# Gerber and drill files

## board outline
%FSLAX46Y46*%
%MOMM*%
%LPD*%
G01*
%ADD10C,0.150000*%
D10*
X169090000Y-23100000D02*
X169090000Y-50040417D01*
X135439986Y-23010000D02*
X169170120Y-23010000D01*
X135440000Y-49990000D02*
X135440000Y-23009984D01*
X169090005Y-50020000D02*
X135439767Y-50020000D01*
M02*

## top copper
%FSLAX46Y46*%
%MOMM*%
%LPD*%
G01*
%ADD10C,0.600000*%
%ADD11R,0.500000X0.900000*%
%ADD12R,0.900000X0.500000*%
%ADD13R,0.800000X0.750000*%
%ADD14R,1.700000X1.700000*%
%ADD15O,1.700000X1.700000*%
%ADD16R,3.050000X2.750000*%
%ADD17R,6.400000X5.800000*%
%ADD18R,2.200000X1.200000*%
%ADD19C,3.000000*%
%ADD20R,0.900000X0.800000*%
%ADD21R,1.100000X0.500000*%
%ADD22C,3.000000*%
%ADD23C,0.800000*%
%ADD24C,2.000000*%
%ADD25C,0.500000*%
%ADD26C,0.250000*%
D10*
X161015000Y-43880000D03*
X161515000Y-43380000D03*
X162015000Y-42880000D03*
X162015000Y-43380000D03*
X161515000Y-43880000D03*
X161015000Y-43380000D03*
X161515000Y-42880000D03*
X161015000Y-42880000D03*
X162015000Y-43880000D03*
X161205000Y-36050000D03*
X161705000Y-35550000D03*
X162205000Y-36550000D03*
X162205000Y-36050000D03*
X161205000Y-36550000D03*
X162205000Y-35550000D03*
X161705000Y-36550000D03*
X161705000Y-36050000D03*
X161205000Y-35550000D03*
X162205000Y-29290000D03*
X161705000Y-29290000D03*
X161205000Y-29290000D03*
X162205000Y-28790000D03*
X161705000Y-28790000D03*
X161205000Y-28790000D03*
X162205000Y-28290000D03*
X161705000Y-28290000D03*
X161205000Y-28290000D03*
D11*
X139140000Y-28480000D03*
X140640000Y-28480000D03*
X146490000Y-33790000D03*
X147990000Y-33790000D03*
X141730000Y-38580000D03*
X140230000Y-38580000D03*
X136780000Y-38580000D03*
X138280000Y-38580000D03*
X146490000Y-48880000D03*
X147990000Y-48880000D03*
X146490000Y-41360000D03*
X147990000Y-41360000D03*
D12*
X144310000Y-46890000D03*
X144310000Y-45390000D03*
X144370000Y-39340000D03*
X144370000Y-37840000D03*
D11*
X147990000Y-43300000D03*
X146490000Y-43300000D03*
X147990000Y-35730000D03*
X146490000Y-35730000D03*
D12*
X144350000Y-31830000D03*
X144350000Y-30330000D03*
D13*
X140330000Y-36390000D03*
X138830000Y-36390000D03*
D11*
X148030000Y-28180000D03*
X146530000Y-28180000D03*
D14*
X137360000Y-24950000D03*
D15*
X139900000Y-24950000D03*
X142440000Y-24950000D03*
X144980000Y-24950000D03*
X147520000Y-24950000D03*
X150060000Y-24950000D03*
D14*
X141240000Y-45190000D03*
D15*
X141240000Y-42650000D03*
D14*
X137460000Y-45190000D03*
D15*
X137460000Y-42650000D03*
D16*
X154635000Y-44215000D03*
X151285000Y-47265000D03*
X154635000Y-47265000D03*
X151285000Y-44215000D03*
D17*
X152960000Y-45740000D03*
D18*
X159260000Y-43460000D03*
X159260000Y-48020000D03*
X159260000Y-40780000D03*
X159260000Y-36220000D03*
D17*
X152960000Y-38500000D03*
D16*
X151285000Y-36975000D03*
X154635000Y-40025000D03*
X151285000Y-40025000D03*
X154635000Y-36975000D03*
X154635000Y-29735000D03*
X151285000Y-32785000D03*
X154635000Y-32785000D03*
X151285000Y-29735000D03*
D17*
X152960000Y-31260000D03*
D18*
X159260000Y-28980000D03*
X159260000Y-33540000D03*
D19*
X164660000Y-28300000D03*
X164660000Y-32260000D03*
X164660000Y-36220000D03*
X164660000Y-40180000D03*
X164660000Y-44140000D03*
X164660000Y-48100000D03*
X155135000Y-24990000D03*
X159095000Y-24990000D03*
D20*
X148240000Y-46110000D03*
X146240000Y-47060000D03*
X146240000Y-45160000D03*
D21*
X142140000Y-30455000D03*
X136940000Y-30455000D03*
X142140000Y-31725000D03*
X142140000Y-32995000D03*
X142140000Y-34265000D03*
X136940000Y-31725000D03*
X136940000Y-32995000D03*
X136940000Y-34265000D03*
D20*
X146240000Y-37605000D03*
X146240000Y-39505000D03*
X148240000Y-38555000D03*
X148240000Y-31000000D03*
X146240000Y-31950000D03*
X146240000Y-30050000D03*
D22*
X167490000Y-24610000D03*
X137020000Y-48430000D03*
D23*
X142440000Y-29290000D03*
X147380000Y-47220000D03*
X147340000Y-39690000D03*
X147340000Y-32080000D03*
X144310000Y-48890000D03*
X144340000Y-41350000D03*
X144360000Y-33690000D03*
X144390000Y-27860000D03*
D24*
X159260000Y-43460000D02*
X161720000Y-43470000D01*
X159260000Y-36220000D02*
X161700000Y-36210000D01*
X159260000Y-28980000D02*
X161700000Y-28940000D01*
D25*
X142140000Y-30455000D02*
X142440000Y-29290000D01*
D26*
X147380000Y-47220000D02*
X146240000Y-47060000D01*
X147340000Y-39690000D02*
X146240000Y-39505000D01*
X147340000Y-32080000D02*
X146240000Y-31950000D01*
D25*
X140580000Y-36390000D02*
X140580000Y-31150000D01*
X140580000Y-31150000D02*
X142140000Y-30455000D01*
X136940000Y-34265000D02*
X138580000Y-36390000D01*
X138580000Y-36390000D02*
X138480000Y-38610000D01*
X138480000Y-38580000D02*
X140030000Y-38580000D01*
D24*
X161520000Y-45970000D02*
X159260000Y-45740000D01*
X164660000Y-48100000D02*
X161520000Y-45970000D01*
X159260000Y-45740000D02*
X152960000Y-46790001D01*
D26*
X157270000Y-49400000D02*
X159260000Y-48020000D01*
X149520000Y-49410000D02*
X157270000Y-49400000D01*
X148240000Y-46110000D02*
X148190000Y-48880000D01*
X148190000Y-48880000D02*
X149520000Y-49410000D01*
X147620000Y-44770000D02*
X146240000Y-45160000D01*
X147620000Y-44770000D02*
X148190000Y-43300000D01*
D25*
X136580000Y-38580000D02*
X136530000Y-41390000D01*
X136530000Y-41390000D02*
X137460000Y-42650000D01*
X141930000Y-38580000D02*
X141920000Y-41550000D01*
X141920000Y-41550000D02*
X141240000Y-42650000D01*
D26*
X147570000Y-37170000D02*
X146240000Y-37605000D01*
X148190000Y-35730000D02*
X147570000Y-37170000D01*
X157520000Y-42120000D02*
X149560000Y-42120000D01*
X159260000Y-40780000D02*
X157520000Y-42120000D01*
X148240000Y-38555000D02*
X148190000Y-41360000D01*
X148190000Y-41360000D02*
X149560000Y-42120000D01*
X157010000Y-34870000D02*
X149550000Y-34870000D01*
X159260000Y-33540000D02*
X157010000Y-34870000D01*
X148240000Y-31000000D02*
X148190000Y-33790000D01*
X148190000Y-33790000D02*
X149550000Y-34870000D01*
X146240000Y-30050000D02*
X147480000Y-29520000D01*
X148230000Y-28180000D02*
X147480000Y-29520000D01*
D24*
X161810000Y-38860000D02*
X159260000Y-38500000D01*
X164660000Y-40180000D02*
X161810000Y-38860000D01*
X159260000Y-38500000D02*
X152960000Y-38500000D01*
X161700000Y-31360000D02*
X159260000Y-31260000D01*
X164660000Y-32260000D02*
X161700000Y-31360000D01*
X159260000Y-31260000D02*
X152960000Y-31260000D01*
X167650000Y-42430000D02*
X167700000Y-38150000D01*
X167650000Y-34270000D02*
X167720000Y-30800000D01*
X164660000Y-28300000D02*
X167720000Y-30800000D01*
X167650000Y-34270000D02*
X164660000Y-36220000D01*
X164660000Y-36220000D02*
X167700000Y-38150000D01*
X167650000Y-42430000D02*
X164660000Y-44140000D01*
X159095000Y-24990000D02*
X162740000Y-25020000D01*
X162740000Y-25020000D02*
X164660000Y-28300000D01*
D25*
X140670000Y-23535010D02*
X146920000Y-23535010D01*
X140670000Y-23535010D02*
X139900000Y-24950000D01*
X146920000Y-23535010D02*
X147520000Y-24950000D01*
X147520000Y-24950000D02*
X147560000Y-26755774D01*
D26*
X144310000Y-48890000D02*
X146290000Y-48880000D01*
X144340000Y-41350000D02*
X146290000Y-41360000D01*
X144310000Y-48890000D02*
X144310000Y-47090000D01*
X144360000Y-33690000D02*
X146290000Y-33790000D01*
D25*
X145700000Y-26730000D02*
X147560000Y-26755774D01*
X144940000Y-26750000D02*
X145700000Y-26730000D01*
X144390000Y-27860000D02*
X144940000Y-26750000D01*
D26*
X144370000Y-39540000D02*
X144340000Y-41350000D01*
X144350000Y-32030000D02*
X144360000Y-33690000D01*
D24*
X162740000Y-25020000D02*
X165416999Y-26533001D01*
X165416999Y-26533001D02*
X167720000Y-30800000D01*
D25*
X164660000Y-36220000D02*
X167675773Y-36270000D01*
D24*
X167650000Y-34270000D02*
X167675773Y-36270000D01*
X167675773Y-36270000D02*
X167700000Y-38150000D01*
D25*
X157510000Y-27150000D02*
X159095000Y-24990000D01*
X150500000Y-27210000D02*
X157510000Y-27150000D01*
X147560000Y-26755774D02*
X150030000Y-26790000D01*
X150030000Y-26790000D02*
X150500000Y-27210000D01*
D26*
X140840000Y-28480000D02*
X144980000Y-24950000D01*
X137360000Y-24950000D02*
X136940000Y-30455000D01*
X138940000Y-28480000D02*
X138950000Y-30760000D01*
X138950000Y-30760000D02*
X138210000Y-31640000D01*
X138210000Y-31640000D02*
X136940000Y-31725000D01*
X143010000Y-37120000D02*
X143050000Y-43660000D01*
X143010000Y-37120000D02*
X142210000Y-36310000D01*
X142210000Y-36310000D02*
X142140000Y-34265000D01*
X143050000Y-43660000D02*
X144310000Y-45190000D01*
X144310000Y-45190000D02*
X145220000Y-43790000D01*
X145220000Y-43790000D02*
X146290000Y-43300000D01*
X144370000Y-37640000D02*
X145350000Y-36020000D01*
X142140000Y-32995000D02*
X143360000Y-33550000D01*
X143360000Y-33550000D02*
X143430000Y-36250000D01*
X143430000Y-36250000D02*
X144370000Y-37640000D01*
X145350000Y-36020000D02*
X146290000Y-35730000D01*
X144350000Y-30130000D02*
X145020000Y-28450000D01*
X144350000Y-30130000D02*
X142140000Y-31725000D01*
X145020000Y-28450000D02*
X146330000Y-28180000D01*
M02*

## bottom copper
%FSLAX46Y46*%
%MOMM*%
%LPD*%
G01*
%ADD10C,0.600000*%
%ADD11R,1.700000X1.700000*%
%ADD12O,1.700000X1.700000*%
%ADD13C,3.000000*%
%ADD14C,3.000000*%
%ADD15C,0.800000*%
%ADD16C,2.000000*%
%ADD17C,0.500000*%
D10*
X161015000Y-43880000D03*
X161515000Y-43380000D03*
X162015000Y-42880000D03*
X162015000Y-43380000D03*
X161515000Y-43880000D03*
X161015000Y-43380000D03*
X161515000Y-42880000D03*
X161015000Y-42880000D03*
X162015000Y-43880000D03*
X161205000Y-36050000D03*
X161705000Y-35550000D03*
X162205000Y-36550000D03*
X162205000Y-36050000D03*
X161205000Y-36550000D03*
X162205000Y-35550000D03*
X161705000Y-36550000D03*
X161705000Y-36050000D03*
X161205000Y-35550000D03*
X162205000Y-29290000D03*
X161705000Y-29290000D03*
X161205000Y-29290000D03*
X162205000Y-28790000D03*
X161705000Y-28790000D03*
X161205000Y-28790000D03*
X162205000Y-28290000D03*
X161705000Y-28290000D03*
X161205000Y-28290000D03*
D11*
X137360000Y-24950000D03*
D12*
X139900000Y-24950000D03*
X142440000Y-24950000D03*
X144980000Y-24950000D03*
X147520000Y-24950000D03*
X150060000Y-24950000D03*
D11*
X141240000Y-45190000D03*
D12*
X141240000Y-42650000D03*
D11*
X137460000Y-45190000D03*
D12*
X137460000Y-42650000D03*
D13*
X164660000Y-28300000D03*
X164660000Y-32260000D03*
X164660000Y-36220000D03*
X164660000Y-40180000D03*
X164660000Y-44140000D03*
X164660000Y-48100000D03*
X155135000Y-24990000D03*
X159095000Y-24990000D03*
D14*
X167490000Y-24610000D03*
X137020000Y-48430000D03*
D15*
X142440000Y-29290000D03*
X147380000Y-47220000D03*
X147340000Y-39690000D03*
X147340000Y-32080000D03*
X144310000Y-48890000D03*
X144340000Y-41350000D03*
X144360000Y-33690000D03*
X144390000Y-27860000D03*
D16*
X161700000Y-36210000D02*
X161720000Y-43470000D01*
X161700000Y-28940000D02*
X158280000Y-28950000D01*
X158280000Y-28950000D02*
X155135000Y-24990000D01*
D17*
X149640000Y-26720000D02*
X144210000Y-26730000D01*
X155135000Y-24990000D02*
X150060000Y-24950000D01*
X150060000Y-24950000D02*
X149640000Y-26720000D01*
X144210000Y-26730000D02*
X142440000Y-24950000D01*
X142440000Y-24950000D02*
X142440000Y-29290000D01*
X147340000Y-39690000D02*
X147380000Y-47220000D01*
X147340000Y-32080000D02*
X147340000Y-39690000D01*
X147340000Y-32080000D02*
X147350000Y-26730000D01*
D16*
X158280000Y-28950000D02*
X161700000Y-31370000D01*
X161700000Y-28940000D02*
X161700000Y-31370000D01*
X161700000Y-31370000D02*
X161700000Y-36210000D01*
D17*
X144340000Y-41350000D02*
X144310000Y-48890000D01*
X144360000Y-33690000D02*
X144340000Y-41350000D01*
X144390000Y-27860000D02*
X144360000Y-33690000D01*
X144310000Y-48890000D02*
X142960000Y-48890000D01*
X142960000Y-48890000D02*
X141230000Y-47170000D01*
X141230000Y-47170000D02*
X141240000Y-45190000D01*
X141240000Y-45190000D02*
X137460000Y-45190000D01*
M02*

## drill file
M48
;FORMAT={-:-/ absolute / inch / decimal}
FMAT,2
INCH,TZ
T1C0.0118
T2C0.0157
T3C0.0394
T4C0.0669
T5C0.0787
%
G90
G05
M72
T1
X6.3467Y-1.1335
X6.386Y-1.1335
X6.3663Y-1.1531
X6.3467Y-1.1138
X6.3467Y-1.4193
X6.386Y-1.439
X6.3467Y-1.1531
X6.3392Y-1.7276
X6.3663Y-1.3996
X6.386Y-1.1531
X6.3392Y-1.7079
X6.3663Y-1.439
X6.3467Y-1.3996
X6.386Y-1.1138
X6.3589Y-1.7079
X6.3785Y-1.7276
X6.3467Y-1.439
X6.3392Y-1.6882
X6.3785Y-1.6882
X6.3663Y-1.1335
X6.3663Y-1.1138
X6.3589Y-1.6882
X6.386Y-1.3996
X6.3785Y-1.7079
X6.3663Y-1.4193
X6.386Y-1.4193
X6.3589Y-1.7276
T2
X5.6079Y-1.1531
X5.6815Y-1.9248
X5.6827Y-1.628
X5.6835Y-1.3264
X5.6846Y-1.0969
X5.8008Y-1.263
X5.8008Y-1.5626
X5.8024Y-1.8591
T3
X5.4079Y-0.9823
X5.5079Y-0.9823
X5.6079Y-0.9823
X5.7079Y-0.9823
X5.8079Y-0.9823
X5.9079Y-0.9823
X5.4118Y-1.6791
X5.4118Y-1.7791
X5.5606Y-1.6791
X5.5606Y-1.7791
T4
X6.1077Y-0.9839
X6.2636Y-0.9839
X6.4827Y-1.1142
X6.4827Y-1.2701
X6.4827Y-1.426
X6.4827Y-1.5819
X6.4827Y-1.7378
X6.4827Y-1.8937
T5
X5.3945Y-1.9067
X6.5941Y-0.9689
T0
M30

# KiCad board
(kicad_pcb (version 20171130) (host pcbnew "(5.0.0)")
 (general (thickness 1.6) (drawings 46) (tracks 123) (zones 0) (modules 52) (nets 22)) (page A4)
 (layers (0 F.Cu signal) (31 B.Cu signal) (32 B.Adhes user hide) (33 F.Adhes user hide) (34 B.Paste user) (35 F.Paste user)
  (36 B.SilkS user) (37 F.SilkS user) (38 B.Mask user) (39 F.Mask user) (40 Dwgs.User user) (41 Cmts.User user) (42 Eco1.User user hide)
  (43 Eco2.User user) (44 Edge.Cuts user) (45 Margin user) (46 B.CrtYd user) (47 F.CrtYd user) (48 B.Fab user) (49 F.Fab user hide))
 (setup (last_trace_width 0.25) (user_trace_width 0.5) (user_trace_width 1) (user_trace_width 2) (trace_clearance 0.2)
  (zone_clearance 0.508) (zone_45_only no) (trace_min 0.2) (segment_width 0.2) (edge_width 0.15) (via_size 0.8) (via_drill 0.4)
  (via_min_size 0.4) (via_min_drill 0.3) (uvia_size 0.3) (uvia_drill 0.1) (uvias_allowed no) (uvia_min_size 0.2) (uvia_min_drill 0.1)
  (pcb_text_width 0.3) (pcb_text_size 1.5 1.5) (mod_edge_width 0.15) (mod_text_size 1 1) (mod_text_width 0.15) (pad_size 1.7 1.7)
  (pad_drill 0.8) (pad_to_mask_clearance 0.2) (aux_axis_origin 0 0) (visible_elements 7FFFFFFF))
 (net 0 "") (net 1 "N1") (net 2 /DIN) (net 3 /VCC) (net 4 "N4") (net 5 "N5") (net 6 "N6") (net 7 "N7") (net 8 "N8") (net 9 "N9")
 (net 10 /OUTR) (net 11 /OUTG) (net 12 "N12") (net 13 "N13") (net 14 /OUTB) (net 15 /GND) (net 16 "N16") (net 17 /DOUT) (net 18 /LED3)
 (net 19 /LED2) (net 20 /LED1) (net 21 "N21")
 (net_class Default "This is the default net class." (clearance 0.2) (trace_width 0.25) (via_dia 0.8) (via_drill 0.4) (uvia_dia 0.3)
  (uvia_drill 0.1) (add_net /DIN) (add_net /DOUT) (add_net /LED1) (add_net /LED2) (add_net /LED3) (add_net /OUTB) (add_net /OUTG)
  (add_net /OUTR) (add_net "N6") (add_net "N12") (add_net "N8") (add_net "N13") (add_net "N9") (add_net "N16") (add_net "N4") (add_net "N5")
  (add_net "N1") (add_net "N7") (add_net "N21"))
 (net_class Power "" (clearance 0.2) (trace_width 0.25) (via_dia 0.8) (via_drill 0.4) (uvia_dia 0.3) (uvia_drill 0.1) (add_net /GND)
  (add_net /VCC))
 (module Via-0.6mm (layer F.Cu) (at 160.99 43.88)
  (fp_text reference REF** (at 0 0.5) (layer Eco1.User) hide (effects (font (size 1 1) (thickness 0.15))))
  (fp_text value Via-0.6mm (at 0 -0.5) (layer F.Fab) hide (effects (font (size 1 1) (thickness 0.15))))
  (pad 1 thru_hole circle (at 0.025 0) (size 0.6 0.6) (drill 0.3) (layers *.Cu) (zone_connect 2)))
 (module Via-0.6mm (layer F.Cu) (at 161.49 43.38)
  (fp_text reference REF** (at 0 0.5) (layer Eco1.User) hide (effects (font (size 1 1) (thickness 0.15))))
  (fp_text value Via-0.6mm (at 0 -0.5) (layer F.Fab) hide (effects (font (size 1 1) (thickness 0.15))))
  (pad 1 thru_hole circle (at 0.025 0) (size 0.6 0.6) (drill 0.3) (layers *.Cu) (zone_connect 2)))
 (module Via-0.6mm (layer F.Cu) (at 161.99 42.88)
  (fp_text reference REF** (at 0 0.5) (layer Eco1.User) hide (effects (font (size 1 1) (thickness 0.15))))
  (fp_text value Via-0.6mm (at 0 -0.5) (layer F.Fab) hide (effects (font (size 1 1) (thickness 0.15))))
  (pad 1 thru_hole circle (at 0.025 0) (size 0.6 0.6) (drill 0.3) (layers *.Cu) (zone_connect 2)))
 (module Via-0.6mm (layer F.Cu) (at 161.99 43.38)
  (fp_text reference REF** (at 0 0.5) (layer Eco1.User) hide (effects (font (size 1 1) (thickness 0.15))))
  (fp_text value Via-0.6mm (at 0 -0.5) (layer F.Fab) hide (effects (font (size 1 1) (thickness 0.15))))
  (pad 1 thru_hole circle (at 0.025 0) (size 0.6 0.6) (drill 0.3) (layers *.Cu) (zone_connect 2)))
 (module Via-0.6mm (layer F.Cu) (at 161.49 43.88)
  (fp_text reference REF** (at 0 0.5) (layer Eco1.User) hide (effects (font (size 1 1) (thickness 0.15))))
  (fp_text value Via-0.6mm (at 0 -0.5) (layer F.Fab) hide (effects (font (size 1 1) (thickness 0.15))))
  (pad 1 thru_hole circle (at 0.025 0) (size 0.6 0.6) (drill 0.3) (layers *.Cu) (zone_connect 2)))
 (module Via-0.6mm (layer F.Cu) (at 160.99 43.38)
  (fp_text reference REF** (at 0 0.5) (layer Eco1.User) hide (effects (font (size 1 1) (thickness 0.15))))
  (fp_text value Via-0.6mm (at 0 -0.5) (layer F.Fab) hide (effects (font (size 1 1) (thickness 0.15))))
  (pad 1 thru_hole circle (at 0.025 0) (size 0.6 0.6) (drill 0.3) (layers *.Cu) (zone_connect 2)))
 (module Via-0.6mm (layer F.Cu) (at 161.49 42.88)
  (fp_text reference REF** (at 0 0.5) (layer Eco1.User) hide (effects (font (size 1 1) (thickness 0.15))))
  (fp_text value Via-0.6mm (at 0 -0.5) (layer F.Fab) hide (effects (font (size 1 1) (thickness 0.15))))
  (pad 1 thru_hole circle (at 0.025 0) (size 0.6 0.6) (drill 0.3) (layers *.Cu) (zone_connect 2)))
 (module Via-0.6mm (layer F.Cu) (at 160.99 42.88)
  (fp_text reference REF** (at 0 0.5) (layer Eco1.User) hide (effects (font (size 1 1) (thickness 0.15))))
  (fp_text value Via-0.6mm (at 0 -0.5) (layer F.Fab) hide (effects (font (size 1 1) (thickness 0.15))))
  (pad 1 thru_hole circle (at 0.025 0) (size 0.6 0.6) (drill 0.3) (layers *.Cu) (zone_connect 2)))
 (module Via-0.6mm (layer F.Cu) (at 161.99 43.88)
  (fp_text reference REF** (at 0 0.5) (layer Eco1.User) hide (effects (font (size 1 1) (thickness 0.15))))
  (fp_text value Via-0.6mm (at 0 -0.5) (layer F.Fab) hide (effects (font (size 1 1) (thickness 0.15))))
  (pad 1 thru_hole circle (at 0.025 0) (size 0.6 0.6) (drill 0.3) (layers *.Cu) (zone_connect 2)))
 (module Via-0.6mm (layer F.Cu) (at 161.18 36.05)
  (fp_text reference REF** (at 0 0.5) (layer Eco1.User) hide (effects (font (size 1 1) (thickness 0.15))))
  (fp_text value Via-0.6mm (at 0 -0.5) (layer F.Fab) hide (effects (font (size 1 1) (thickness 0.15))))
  (pad 1 thru_hole circle (at 0.025 0) (size 0.6 0.6) (drill 0.3) (layers *.Cu) (zone_connect 2)))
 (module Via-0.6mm (layer F.Cu) (at 161.68 35.55)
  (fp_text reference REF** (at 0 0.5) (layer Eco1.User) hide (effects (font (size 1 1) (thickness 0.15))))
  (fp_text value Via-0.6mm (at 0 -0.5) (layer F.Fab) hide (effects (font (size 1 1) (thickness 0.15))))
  (pad 1 thru_hole circle (at 0.025 0) (size 0.6 0.6) (drill 0.3) (layers *.Cu) (zone_connect 2)))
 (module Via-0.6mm (layer F.Cu) (at 162.18 36.55)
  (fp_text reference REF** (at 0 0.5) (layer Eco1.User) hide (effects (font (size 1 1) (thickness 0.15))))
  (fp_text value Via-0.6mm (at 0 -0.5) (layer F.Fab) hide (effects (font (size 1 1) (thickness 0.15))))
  (pad 1 thru_hole circle (at 0.025 0) (size 0.6 0.6) (drill 0.3) (layers *.Cu) (zone_connect 2)))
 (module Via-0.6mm (layer F.Cu) (at 162.18 36.05)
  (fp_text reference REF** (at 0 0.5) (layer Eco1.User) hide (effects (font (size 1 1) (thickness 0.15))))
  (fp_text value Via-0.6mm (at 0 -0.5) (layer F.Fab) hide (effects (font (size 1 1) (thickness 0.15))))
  (pad 1 thru_hole circle (at 0.025 0) (size 0.6 0.6) (drill 0.3) (layers *.Cu) (zone_connect 2)))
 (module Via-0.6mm (layer F.Cu) (at 161.18 36.55)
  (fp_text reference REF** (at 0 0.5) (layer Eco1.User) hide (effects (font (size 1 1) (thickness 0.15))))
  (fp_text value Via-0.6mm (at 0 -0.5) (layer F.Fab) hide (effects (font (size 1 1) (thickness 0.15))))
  (pad 1 thru_hole circle (at 0.025 0) (size 0.6 0.6) (drill 0.3) (layers *.Cu) (zone_connect 2)))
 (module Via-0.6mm (layer F.Cu) (at 162.18 35.55)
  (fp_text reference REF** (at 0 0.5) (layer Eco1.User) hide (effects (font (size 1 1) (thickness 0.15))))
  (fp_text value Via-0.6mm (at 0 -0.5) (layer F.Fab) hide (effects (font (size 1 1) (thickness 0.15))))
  (pad 1 thru_hole circle (at 0.025 0) (size 0.6 0.6) (drill 0.3) (layers *.Cu) (zone_connect 2)))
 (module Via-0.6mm (layer F.Cu) (at 161.68 36.55)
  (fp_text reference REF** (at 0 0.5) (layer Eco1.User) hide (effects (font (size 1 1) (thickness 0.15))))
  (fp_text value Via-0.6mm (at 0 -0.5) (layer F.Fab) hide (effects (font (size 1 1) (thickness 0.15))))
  (pad 1 thru_hole circle (at 0.025 0) (size 0.6 0.6) (drill 0.3) (layers *.Cu) (zone_connect 2)))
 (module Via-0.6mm (layer F.Cu) (at 161.68 36.05)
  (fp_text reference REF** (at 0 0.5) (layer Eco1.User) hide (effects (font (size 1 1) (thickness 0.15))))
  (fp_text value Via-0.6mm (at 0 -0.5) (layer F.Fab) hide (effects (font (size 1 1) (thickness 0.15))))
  (pad 1 thru_hole circle (at 0.025 0) (size 0.6 0.6) (drill 0.3) (layers *.Cu) (zone_connect 2)))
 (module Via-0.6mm (layer F.Cu) (at 161.18 35.55)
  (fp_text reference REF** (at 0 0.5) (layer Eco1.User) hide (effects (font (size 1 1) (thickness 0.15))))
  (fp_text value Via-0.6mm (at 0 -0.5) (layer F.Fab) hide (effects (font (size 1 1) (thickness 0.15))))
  (pad 1 thru_hole circle (at 0.025 0) (size 0.6 0.6) (drill 0.3) (layers *.Cu) (zone_connect 2)))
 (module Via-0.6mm (layer F.Cu) (at 162.18 29.29)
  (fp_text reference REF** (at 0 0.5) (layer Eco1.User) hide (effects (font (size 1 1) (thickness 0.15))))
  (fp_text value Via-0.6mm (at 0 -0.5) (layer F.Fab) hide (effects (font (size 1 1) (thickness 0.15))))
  (pad 1 thru_hole circle (at 0.025 0) (size 0.6 0.6) (drill 0.3) (layers *.Cu) (zone_connect 2)))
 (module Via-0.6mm (layer F.Cu) (at 161.68 29.29)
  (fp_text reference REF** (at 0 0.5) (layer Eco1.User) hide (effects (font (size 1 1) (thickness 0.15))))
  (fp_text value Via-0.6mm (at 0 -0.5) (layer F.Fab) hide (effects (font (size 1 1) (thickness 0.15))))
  (pad 1 thru_hole circle (at 0.025 0) (size 0.6 0.6) (drill 0.3) (layers *.Cu) (zone_connect 2)))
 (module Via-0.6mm (layer F.Cu) (at 161.18 29.29)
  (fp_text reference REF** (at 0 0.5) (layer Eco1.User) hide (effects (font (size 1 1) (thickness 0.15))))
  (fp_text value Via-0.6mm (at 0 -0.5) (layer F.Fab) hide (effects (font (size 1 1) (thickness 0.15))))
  (pad 1 thru_hole circle (at 0.025 0) (size 0.6 0.6) (drill 0.3) (layers *.Cu) (zone_connect 2)))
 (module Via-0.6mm (layer F.Cu) (at 162.18 28.79)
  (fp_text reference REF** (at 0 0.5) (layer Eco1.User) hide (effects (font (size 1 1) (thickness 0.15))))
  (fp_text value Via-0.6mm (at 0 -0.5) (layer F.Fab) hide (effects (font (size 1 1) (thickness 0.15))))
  (pad 1 thru_hole circle (at 0.025 0) (size 0.6 0.6) (drill 0.3) (layers *.Cu) (zone_connect 2)))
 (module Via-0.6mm (layer F.Cu) (at 161.68 28.79)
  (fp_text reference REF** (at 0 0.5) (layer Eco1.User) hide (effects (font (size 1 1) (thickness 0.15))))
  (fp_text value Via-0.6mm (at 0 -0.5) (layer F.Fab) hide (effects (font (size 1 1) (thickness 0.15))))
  (pad 1 thru_hole circle (at 0.025 0) (size 0.6 0.6) (drill 0.3) (layers *.Cu) (zone_connect 2)))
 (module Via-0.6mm (layer F.Cu) (at 161.18 28.79)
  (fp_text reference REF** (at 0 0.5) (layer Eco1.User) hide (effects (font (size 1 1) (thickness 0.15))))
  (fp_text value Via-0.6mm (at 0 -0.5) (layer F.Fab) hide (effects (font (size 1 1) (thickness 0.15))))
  (pad 1 thru_hole circle (at 0.025 0) (size 0.6 0.6) (drill 0.3) (layers *.Cu) (zone_connect 2)))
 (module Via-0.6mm (layer F.Cu) (at 162.18 28.29)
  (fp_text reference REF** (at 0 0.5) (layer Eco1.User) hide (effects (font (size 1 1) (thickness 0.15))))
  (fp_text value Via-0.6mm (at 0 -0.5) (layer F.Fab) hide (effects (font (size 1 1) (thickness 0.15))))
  (pad 1 thru_hole circle (at 0.025 0) (size 0.6 0.6) (drill 0.3) (layers *.Cu) (zone_connect 2)))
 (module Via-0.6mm (layer F.Cu) (at 161.68 28.29)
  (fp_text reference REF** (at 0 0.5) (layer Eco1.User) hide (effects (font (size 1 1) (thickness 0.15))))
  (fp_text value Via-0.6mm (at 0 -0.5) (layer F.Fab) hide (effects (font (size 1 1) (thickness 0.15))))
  (pad 1 thru_hole circle (at 0.025 0) (size 0.6 0.6) (drill 0.3) (layers *.Cu) (zone_connect 2)))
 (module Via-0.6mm (layer F.Cu) (at 161.18 28.29)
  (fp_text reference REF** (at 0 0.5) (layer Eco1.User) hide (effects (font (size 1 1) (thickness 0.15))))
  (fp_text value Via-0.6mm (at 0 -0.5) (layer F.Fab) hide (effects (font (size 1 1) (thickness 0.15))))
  (pad 1 thru_hole circle (at 0.025 0) (size 0.6 0.6) (drill 0.3) (layers *.Cu) (zone_connect 2)))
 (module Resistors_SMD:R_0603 (layer F.Cu) (at 139.89 28.48)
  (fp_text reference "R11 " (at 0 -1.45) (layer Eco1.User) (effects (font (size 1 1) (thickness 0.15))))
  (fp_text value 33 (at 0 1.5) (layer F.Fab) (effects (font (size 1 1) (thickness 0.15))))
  (pad 1 smd rect (at -0.75 0) (size 0.5 0.9) (layers F.Cu F.Paste F.Mask) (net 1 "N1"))
  (pad 2 smd rect (at 0.75 0) (size 0.5 0.9) (layers F.Cu F.Paste F.Mask) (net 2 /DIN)))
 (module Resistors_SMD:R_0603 (layer F.Cu) (at 147.24 33.79)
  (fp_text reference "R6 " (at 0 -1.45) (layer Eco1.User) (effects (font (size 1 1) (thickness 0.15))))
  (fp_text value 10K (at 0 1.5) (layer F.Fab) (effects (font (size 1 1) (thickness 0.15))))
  (pad 1 smd rect (at -0.75 0) (size 0.5 0.9) (layers F.Cu F.Paste F.Mask) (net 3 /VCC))
  (pad 2 smd rect (at 0.75 0) (size 0.5 0.9) (layers F.Cu F.Paste F.Mask) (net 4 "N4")))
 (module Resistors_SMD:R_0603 (layer F.Cu) (at 140.98 38.58 180)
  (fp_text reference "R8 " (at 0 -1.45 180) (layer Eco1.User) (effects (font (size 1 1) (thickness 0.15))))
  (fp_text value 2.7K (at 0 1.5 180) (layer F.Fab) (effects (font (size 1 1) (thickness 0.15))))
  (pad 1 smd rect (at -0.75 0 180) (size 0.5 0.9) (layers F.Cu F.Paste F.Mask) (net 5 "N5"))
  (pad 2 smd rect (at 0.75 0 180) (size 0.5 0.9) (layers F.Cu F.Paste F.Mask) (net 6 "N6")))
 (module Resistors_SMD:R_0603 (layer F.Cu) (at 137.53 38.58)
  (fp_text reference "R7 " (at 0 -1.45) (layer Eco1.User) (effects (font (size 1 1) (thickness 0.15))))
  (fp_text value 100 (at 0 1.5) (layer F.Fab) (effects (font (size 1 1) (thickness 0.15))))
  (pad 1 smd rect (at -0.75 0) (size 0.5 0.9) (layers F.Cu F.Paste F.Mask) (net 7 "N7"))
  (pad 2 smd rect (at 0.75 0) (size 0.5 0.9) (layers F.Cu F.Paste F.Mask) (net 6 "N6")))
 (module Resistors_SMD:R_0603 (layer F.Cu) (at 147.24 48.88)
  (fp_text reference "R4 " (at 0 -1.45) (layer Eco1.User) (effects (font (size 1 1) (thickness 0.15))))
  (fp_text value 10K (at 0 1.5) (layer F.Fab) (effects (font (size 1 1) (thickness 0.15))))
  (pad 1 smd rect (at -0.75 0) (size 0.5 0.9) (layers F.Cu F.Paste F.Mask) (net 3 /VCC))
  (pad 2 smd rect (at 0.75 0) (size 0.5 0.9) (layers F.Cu F.Paste F.Mask) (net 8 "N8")))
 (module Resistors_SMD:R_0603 (layer F.Cu) (at 147.24 41.36)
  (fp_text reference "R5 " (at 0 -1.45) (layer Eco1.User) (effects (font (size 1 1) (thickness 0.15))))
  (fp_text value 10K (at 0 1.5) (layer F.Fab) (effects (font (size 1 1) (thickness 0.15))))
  (pad 1 smd rect (at -0.75 0) (size 0.5 0.9) (layers F.Cu F.Paste F.Mask) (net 3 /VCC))
  (pad 2 smd rect (at 0.75 0) (size 0.5 0.9) (layers F.Cu F.Paste F.Mask) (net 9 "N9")))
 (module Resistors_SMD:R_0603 (layer F.Cu) (at 144.31 46.14 90)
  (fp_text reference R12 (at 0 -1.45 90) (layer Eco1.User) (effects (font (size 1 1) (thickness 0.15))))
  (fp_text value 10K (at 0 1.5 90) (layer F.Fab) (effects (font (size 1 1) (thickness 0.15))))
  (pad 1 smd rect (at -0.75 0 90) (size 0.5 0.9) (layers F.Cu F.Paste F.Mask) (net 3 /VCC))
  (pad 2 smd rect (at 0.75 0 90) (size 0.5 0.9) (layers F.Cu F.Paste F.Mask) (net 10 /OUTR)))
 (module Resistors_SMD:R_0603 (layer F.Cu) (at 144.37 38.59 90)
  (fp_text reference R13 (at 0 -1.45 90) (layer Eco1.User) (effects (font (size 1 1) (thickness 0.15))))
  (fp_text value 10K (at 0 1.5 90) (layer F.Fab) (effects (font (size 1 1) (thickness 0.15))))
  (pad 1 smd rect (at -0.75 0 90) (size 0.5 0.9) (layers F.Cu F.Paste F.Mask) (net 3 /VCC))
  (pad 2 smd rect (at 0.75 0 90) (size 0.5 0.9) (layers F.Cu F.Paste F.Mask) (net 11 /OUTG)))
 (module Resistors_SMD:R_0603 (layer F.Cu) (at 147.24 43.3 180)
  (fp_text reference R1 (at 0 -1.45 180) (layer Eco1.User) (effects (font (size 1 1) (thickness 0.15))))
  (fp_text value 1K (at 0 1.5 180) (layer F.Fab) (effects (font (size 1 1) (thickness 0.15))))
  (pad 1 smd rect (at -0.75 0 180) (size 0.5 0.9) (layers F.Cu F.Paste F.Mask) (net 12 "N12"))
  (pad 2 smd rect (at 0.75 0 180) (size 0.5 0.9) (layers F.Cu F.Paste F.Mask) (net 10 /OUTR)))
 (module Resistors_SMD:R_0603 (layer F.Cu) (at 147.24 35.73 180)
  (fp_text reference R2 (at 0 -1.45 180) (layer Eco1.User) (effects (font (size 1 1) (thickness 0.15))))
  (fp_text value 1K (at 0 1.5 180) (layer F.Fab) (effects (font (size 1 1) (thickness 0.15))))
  (pad 1 smd rect (at -0.75 0 180) (size 0.5 0.9) (layers F.Cu F.Paste F.Mask) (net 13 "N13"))
  (pad 2 smd rect (at 0.75 0 180) (size 0.5 0.9) (layers F.Cu F.Paste F.Mask) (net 11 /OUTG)))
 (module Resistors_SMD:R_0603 (layer F.Cu) (at 144.35 31.08 90)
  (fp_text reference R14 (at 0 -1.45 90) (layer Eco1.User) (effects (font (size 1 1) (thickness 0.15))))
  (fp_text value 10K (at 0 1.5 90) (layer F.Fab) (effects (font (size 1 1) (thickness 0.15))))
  (pad 1 smd rect (at -0.75 0 90) (size 0.5 0.9) (layers F.Cu F.Paste F.Mask) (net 3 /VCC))
  (pad 2 smd rect (at 0.75 0 90) (size 0.5 0.9) (layers F.Cu F.Paste F.Mask) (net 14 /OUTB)))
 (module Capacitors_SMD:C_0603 (layer F.Cu) (at 139.58 36.39)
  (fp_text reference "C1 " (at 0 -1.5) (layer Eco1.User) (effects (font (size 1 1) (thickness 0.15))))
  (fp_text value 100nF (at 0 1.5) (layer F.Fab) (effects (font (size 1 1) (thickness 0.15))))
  (pad 2 smd rect (at 0.75 0) (size 0.8 0.75) (layers F.Cu F.Paste F.Mask) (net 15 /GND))
  (pad 1 smd rect (at -0.75 0) (size 0.8 0.75) (layers F.Cu F.Paste F.Mask) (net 6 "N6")))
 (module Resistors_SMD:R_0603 (layer F.Cu) (at 147.28 28.18 180)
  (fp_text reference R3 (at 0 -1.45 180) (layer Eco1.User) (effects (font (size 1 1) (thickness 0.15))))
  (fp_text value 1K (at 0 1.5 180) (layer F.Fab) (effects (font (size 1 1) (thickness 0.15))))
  (pad 1 smd rect (at -0.75 0 180) (size 0.5 0.9) (layers F.Cu F.Paste F.Mask) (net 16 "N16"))
  (pad 2 smd rect (at 0.75 0 180) (size 0.5 0.9) (layers F.Cu F.Paste F.Mask) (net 14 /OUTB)))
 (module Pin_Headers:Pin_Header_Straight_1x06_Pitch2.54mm (layer F.Cu) (at 137.36 24.95 90)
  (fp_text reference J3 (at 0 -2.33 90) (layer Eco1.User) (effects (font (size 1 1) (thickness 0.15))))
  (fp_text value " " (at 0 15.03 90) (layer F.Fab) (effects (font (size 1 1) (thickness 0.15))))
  (pad 1 thru_hole rect (at 0 0 90) (size 1.7 1.7) (drill 1) (layers *.Cu *.Mask) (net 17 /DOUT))
  (pad 2 thru_hole oval (at 0 2.54 90) (size 1.7 1.7) (drill 1) (layers *.Cu *.Mask) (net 3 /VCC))
  (pad 3 thru_hole oval (at 0 5.08 90) (size 1.7 1.7) (drill 1) (layers *.Cu *.Mask) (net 15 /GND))
  (pad 4 thru_hole oval (at 0 7.62 90) (size 1.7 1.7) (drill 1) (layers *.Cu *.Mask) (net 2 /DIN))
  (pad 5 thru_hole oval (at 0 10.16 90) (size 1.7 1.7) (drill 1) (layers *.Cu *.Mask) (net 3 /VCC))
  (pad 6 thru_hole oval (at 0 12.7 90) (size 1.7 1.7) (drill 1) (layers *.Cu *.Mask) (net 15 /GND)))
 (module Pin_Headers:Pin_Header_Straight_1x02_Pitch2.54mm (layer F.Cu) (at 141.24 45.19 180)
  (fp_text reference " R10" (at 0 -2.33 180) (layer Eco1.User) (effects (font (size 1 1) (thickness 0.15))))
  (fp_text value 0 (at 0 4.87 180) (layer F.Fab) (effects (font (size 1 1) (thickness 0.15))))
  (pad 1 thru_hole rect (at 0 0 180) (size 1.7 1.7) (drill 1) (layers *.Cu *.Mask) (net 3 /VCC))
  (pad 2 thru_hole oval (at 0 2.54 180) (size 1.7 1.7) (drill 1) (layers *.Cu *.Mask) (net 5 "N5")))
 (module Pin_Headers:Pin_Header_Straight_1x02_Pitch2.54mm (layer F.Cu) (at 137.46 45.19 180)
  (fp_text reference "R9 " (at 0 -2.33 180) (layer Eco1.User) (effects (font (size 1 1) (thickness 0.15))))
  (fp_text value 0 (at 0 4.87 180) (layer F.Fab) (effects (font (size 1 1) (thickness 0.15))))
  (pad 1 thru_hole rect (at 0 0 180) (size 1.7 1.7) (drill 1) (layers *.Cu *.Mask) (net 3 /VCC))
  (pad 2 thru_hole oval (at 0 2.54 180) (size 1.7 1.7) (drill 1) (layers *.Cu *.Mask) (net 7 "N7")))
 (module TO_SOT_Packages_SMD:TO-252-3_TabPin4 (layer F.Cu) (at 155.06 45.74 180)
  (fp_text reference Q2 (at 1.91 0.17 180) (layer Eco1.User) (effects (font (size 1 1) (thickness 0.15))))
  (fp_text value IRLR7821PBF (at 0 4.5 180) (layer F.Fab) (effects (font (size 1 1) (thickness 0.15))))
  (pad 4 smd rect (at 0.425 1.525 180) (size 3.05 2.75) (layers F.Cu F.Paste))
  (pad 4 smd rect (at 3.775 -1.525 180) (size 3.05 2.75) (layers F.Cu F.Paste))
  (pad 4 smd rect (at 0.425 -1.525 180) (size 3.05 2.75) (layers F.Cu F.Paste))
  (pad 4 smd rect (at 3.775 1.525 180) (size 3.05 2.75) (layers F.Cu F.Paste))
  (pad 4 smd rect (at 2.1 0 180) (size 6.4 5.8) (layers F.Cu F.Mask))
  (pad 3 smd rect (at -4.2 2.28 180) (size 2.2 1.2) (layers F.Cu F.Paste F.Mask) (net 15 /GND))
  (pad 1 smd rect (at -4.2 -2.28 180) (size 2.2 1.2) (layers F.Cu F.Paste F.Mask) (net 8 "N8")))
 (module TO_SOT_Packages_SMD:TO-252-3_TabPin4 (layer F.Cu) (at 155.06 38.5 180)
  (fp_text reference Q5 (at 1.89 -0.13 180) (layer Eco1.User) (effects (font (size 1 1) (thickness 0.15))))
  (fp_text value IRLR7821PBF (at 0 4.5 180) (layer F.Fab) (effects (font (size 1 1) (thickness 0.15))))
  (pad 1 smd rect (at -4.2 -2.28 180) (size 2.2 1.2) (layers F.Cu F.Paste F.Mask) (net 9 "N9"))
  (pad 3 smd rect (at -4.2 2.28 180) (size 2.2 1.2) (layers F.Cu F.Paste F.Mask) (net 15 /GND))
  (pad 4 smd rect (at 2.1 0 180) (size 6.4 5.8) (layers F.Cu F.Mask))
  (pad 4 smd rect (at 3.775 1.525 180) (size 3.05 2.75) (layers F.Cu F.Paste))
  (pad 4 smd rect (at 0.425 -1.525 180) (size 3.05 2.75) (layers F.Cu F.Paste))
  (pad 4 smd rect (at 3.775 -1.525 180) (size 3.05 2.75) (layers F.Cu F.Paste))
  (pad 4 smd rect (at 0.425 1.525 180) (size 3.05 2.75) (layers F.Cu F.Paste)))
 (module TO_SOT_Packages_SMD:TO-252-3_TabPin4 (layer F.Cu) (at 155.06 31.26 180)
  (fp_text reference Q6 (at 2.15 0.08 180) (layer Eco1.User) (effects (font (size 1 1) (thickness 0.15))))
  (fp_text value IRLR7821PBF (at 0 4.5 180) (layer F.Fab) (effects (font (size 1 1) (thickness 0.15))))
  (pad 4 smd rect (at 0.425 1.525 180) (size 3.05 2.75) (layers F.Cu F.Paste))
  (pad 4 smd rect (at 3.775 -1.525 180) (size 3.05 2.75) (layers F.Cu F.Paste))
  (pad 4 smd rect (at 0.425 -1.525 180) (size 3.05 2.75) (layers F.Cu F.Paste))
  (pad 4 smd rect (at 3.775 1.525 180) (size 3.05 2.75) (layers F.Cu F.Paste))
  (pad 4 smd rect (at 2.1 0 180) (size 6.4 5.8) (layers F.Cu F.Mask))
  (pad 3 smd rect (at -4.2 2.28 180) (size 2.2 1.2) (layers F.Cu F.Paste F.Mask) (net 15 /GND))
  (pad 1 smd rect (at -4.2 -2.28 180) (size 2.2 1.2) (layers F.Cu F.Paste F.Mask) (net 4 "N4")))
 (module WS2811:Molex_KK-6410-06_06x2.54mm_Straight (layer F.Cu) (at 164.66 48.1 90)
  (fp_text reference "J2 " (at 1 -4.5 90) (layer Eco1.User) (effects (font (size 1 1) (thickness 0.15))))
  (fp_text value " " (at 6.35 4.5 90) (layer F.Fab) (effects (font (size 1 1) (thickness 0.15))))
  (pad 6 thru_hole circle (at 19.8 0 90) (size 3 3) (drill 1.7) (layers *.Cu *.Mask) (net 3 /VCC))
  (pad 5 thru_hole circle (at 15.84 0 90) (size 3 3) (drill 1.7) (layers *.Cu *.Mask) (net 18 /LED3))
  (pad 4 thru_hole circle (at 11.88 0 90) (size 3 3) (drill 1.7) (layers *.Cu *.Mask) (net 3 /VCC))
  (pad 3 thru_hole circle (at 7.92 0 90) (size 3 3) (drill 1.7) (layers *.Cu *.Mask) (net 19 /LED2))
  (pad 2 thru_hole circle (at 3.96 0 90) (size 3 3) (drill 1.7) (layers *.Cu *.Mask) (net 3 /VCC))
  (pad 1 thru_hole circle (at 0 0 90) (size 3 3) (drill 1.7) (layers *.Cu *.Mask) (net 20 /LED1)))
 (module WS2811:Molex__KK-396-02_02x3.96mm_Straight (layer F.Cu) (at 159.07 24.99 180)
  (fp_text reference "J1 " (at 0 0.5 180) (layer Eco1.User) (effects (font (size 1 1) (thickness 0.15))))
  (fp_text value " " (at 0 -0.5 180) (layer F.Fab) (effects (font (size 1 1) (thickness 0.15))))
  (pad 2 thru_hole circle (at 3.935 0 180) (size 3 3) (drill 1.7) (layers *.Cu *.Mask) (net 15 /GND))
  (pad 1 thru_hole circle (at -0.025 0 180) (size 3 3) (drill 1.7) (layers *.Cu *.Mask) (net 3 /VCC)))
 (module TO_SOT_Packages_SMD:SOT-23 (layer F.Cu) (at 147.24 46.11)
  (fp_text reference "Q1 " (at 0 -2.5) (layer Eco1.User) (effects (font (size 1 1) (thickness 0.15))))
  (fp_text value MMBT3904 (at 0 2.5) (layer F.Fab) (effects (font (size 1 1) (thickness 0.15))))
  (pad 3 smd rect (at 1 0) (size 0.9 0.8) (layers F.Cu F.Paste F.Mask) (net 8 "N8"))
  (pad 2 smd rect (at -1 0.95) (size 0.9 0.8) (layers F.Cu F.Paste F.Mask) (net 15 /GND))
  (pad 1 smd rect (at -1 -0.95) (size 0.9 0.8) (layers F.Cu F.Paste F.Mask) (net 12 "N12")))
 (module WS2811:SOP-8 (layer F.Cu) (at 139.54 32.36 90)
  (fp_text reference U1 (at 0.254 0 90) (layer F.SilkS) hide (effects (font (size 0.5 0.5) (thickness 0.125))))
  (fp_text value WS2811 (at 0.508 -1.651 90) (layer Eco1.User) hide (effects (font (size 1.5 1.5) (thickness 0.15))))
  (pad 4 smd rect (at 1.905 2.6 90) (size 0.5 1.1) (layers F.Cu F.Paste F.Mask) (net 15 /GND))
  (pad 5 smd rect (at 1.905 -2.6 90) (size 0.5 1.1) (layers F.Cu F.Paste F.Mask) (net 17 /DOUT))
  (pad 3 smd rect (at 0.635 2.6 90) (size 0.5 1.1) (layers F.Cu F.Paste F.Mask) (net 14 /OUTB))
  (pad 2 smd rect (at -0.635 2.6 90) (size 0.5 1.1) (layers F.Cu F.Paste F.Mask) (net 11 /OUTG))
  (pad 1 smd rect (at -1.905 2.6 90) (size 0.5 1.1) (layers F.Cu F.Paste F.Mask) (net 10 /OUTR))
  (pad 6 smd rect (at 0.635 -2.6 90) (size 0.5 1.1) (layers F.Cu F.Paste F.Mask) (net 1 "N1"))
  (pad 7 smd rect (at -0.635 -2.6 90) (size 0.5 1.1) (layers F.Cu F.Paste F.Mask) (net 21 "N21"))
  (pad 8 smd rect (at -1.905 -2.6 90) (size 0.5 1.1) (layers F.Cu F.Paste F.Mask) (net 6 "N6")))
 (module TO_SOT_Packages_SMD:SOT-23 (layer F.Cu) (at 147.24 38.555)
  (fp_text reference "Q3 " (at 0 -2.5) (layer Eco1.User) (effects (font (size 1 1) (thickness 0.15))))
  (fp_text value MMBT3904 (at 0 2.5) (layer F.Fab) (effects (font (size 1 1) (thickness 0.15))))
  (pad 1 smd rect (at -1 -0.95) (size 0.9 0.8) (layers F.Cu F.Paste F.Mask) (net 13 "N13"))
  (pad 2 smd rect (at -1 0.95) (size 0.9 0.8) (layers F.Cu F.Paste F.Mask) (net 15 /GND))
  (pad 3 smd rect (at 1 0) (size 0.9 0.8) (layers F.Cu F.Paste F.Mask) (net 9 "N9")))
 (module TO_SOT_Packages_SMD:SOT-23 (layer F.Cu) (at 147.24 31)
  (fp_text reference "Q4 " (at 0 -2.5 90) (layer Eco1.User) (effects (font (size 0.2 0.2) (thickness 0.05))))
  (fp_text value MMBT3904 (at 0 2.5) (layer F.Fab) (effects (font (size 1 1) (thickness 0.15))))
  (pad 3 smd rect (at 1 0) (size 0.9 0.8) (layers F.Cu F.Paste F.Mask) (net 4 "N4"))
  (pad 2 smd rect (at -1 0.95) (size 0.9 0.8) (layers F.Cu F.Paste F.Mask) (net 15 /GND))
  (pad 1 smd rect (at -1 -0.95) (size 0.9 0.8) (layers F.Cu F.Paste F.Mask) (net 16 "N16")))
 (gr_line (start 169.09 23.1) (end 169.09 50.040417) (layer Edge.Cuts) (width 0.15))
 (gr_line (start 135.439986 23.01) (end 169.17012 23.01) (layer Edge.Cuts) (width 0.15))
 (gr_line (start 135.44 49.99) (end 135.44 23.009984) (layer Edge.Cuts) (width 0.15))
 (gr_line (start 169.090005 50.02) (end 135.439767 50.02) (layer Edge.Cuts) (width 0.15))
 (via (at 167.49 24.61) (size 3) (drill 2) (layers F.Cu B.Cu) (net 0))
 (via (at 137.02 48.43) (size 3) (drill 2) (layers F.Cu B.Cu) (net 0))
 (segment (start 161.7 36.21) (end 161.72 43.47) (width 2) (layer B.Cu) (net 15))
 (segment (start 159.26 43.46) (end 161.72 43.47) (width 2) (layer F.Cu) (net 15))
 (segment (start 159.26 36.22) (end 161.7 36.21) (width 2) (layer F.Cu) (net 15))
 (segment (start 159.26 28.98) (end 161.7 28.94) (width 2) (layer F.Cu) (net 15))
 (segment (start 161.7 28.94) (end 158.28 28.95) (width 2) (layer B.Cu) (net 15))
 (segment (start 158.28 28.95) (end 155.135 24.99) (width 2) (layer B.Cu) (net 15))
 (via (at 142.44 29.29) (size 0.8) (drill 0.4) (layers F.Cu B.Cu) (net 15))
 (segment (start 142.14 30.455) (end 142.44 29.29) (width 0.5) (layer F.Cu) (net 15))
 (segment (start 149.64 26.72) (end 144.21 26.73) (width 0.5) (layer B.Cu) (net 15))
 (segment (start 155.135 24.99) (end 150.06 24.95) (width 0.5) (layer B.Cu) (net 15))
 (segment (start 150.06 24.95) (end 149.64 26.72) (width 0.5) (layer B.Cu) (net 15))
 (segment (start 144.21 26.73) (end 142.44 24.95) (width 0.5) (layer B.Cu) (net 15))
 (segment (start 142.44 24.95) (end 142.44 29.29) (width 0.5) (layer B.Cu) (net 15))
 (via (at 147.38 47.22) (size 0.8) (drill 0.4) (layers F.Cu B.Cu) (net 15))
 (segment (start 147.38 47.22) (end 146.24 47.06) (width 0.25) (layer F.Cu) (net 15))
 (via (at 147.34 39.69) (size 0.8) (drill 0.4) (layers F.Cu B.Cu) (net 15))
 (segment (start 147.34 39.69) (end 147.38 47.22) (width 0.5) (layer B.Cu) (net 15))
 (segment (start 147.34 39.69) (end 146.24 39.505) (width 0.25) (layer F.Cu) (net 15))
 (via (at 147.34 32.08) (size 0.8) (drill 0.4) (layers F.Cu B.Cu) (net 15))
 (segment (start 147.34 32.08) (end 147.34 39.69) (width 0.5) (layer B.Cu) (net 15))
 (segment (start 147.34 32.08) (end 147.35 26.73) (width 0.5) (layer B.Cu) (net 15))
 (segment (start 147.34 32.08) (end 146.24 31.95) (width 0.25) (layer F.Cu) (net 15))
 (segment (start 158.28 28.95) (end 161.7 31.37) (width 2) (layer B.Cu) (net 15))
 (segment (start 161.7 28.94) (end 161.7 31.37) (width 2) (layer B.Cu) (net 15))
 (segment (start 161.7 31.37) (end 161.7 36.21) (width 2) (layer B.Cu) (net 15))
 (segment (start 140.58 36.39) (end 140.58 31.15) (width 0.5) (layer F.Cu) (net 15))
 (segment (start 140.58 31.15) (end 142.14 30.455) (width 0.5) (layer F.Cu) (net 15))
 (segment (start 136.94 34.265) (end 138.58 36.39) (width 0.5) (layer F.Cu) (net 6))
 (segment (start 138.58 36.39) (end 138.48 38.61) (width 0.5) (layer F.Cu) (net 6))
 (segment (start 138.48 38.58) (end 140.03 38.58) (width 0.5) (layer F.Cu) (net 6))
 (segment (start 161.52 45.97) (end 159.26 45.74) (width 2) (layer F.Cu) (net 20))
 (segment (start 164.66 48.1) (end 161.52 45.97) (width 2) (layer F.Cu) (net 20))
 (segment (start 159.26 45.74) (end 152.96 46.790001) (width 2) (layer F.Cu) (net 20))
 (segment (start 157.27 49.4) (end 159.26 48.02) (width 0.25) (layer F.Cu) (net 8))
 (segment (start 149.52 49.41) (end 157.27 49.4) (width 0.25) (layer F.Cu) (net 8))
 (segment (start 148.24 46.11) (end 148.19 48.88) (width 0.25) (layer F.Cu) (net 8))
 (segment (start 148.19 48.88) (end 149.52 49.41) (width 0.25) (layer F.Cu) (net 8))
 (segment (start 147.62 44.77) (end 146.24 45.16) (width 0.25) (layer F.Cu) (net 12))
 (segment (start 147.62 44.77) (end 148.19 43.3) (width 0.25) (layer F.Cu) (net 12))
 (segment (start 136.58 38.58) (end 136.53 41.39) (width 0.5) (layer F.Cu) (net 7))
 (segment (start 136.53 41.39) (end 137.46 42.65) (width 0.5) (layer F.Cu) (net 7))
 (segment (start 141.93 38.58) (end 141.92 41.55) (width 0.5) (layer F.Cu) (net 5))
 (segment (start 141.92 41.55) (end 141.24 42.65) (width 0.5) (layer F.Cu) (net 5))
 (segment (start 147.57 37.17) (end 146.24 37.605) (width 0.25) (layer F.Cu) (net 13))
 (segment (start 148.19 35.73) (end 147.57 37.17) (width 0.25) (layer F.Cu) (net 13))
 (segment (start 157.52 42.12) (end 149.56 42.12) (width 0.25) (layer F.Cu) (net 9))
 (segment (start 159.26 40.78) (end 157.52 42.12) (width 0.25) (layer F.Cu) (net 9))
 (segment (start 148.24 38.555) (end 148.19 41.36) (width 0.25) (layer F.Cu) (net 9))
 (segment (start 148.19 41.36) (end 149.56 42.12) (width 0.25) (layer F.Cu) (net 9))
 (segment (start 157.01 34.87) (end 149.55 34.87) (width 0.25) (layer F.Cu) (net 4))
 (segment (start 159.26 33.54) (end 157.01 34.87) (width 0.25) (layer F.Cu) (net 4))
 (segment (start 148.24 31) (end 148.19 33.79) (width 0.25) (layer F.Cu) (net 4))
 (segment (start 148.19 33.79) (end 149.55 34.87) (width 0.25) (layer F.Cu) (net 4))
 (segment (start 146.24 30.05) (end 147.48 29.52) (width 0.25) (layer F.Cu) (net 16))
 (segment (start 148.23 28.18) (end 147.48 29.52) (width 0.25) (layer F.Cu) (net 16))
 (segment (start 161.81 38.86) (end 159.26 38.5) (width 2) (layer F.Cu) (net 19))
 (segment (start 164.66 40.18) (end 161.81 38.86) (width 2) (layer F.Cu) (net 19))
 (segment (start 159.26 38.5) (end 152.96 38.5) (width 2) (layer F.Cu) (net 19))
 (segment (start 161.7 31.36) (end 159.26 31.26) (width 2) (layer F.Cu) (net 18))
 (segment (start 164.66 32.26) (end 161.7 31.36) (width 2) (layer F.Cu) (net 18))
 (segment (start 159.26 31.26) (end 152.96 31.26) (width 2) (layer F.Cu) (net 18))
 (segment (start 167.65 42.43) (end 167.7 38.15) (width 2) (layer F.Cu) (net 3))
 (segment (start 167.65 34.27) (end 167.72 30.8) (width 2) (layer F.Cu) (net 3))
 (segment (start 164.66 28.3) (end 167.72 30.8) (width 2) (layer F.Cu) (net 3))
 (segment (start 167.65 34.27) (end 164.66 36.22) (width 2) (layer F.Cu) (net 3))
 (segment (start 164.66 36.22) (end 167.7 38.15) (width 2) (layer F.Cu) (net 3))
 (segment (start 167.65 42.43) (end 164.66 44.14) (width 2) (layer F.Cu) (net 3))
 (segment (start 159.095 24.99) (end 162.74 25.02) (width 2) (layer F.Cu) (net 3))
 (segment (start 162.74 25.02) (end 164.66 28.3) (width 2) (layer F.Cu) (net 3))
 (segment (start 140.67 23.53501) (end 146.92 23.53501) (width 0.5) (layer F.Cu) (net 3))
 (segment (start 140.67 23.53501) (end 139.9 24.95) (width 0.5) (layer F.Cu) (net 3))
 (segment (start 146.92 23.53501) (end 147.52 24.95) (width 0.5) (layer F.Cu) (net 3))
 (segment (start 147.52 24.95) (end 147.56 26.755774) (width 0.5) (layer F.Cu) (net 3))
 (segment (start 144.31 48.89) (end 146.29 48.88) (width 0.25) (layer F.Cu) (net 3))
 (via (at 144.31 48.89) (size 0.8) (drill 0.4) (layers F.Cu B.Cu) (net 3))
 (segment (start 144.34 41.35) (end 146.29 41.36) (width 0.25) (layer F.Cu) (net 3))
 (via (at 144.34 41.35) (size 0.8) (drill 0.4) (layers F.Cu B.Cu) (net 3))
 (segment (start 144.34 41.35) (end 144.31 48.89) (width 0.5) (layer B.Cu) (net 3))
 (segment (start 144.31 48.89) (end 144.31 47.09) (width 0.25) (layer F.Cu) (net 3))
 (via (at 144.36 33.69) (size 0.8) (drill 0.4) (layers F.Cu B.Cu) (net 3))
 (segment (start 144.36 33.69) (end 144.34 41.35) (width 0.5) (layer B.Cu) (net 3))
 (segment (start 144.36 33.69) (end 146.29 33.79) (width 0.25) (layer F.Cu) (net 3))
 (via (at 144.39 27.86) (size 0.8) (drill 0.4) (layers F.Cu B.Cu) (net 3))
 (segment (start 144.39 27.86) (end 144.36 33.69) (width 0.5) (layer B.Cu) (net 3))
 (segment (start 145.7 26.73) (end 147.56 26.755774) (width 0.5) (layer F.Cu) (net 3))
 (segment (start 144.94 26.75) (end 145.7 26.73) (width 0.5) (layer F.Cu) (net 3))
 (segment (start 144.39 27.86) (end 144.94 26.75) (width 0.5) (layer F.Cu) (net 3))
 (segment (start 144.37 39.54) (end 144.34 41.35) (width 0.25) (layer F.Cu) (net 3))
 (segment (start 144.35 32.03) (end 144.36 33.69) (width 0.25) (layer F.Cu) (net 3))
 (segment (start 162.74 25.02) (end 165.416999 26.533001) (width 2) (layer F.Cu) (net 3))
 (segment (start 165.416999 26.533001) (end 167.72 30.8) (width 2) (layer F.Cu) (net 3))
 (segment (start 164.66 36.22) (end 167.675773 36.27) (width 0.5) (layer F.Cu) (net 3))
 (segment (start 167.65 34.27) (end 167.675773 36.27) (width 2) (layer F.Cu) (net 3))
 (segment (start 167.675773 36.27) (end 167.7 38.15) (width 2) (layer F.Cu) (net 3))
 (segment (start 144.31 48.89) (end 142.96 48.89) (width 0.5) (layer B.Cu) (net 3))
 (segment (start 142.96 48.89) (end 141.23 47.17) (width 0.5) (layer B.Cu) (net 3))
 (segment (start 141.23 47.17) (end 141.24 45.19) (width 0.5) (layer B.Cu) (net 3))
 (segment (start 141.24 45.19) (end 137.46 45.19) (width 0.5) (layer B.Cu) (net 3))
 (segment (start 157.51 27.15) (end 159.095 24.99) (width 0.5) (layer F.Cu) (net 3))
 (segment (start 150.5 27.21) (end 157.51 27.15) (width 0.5) (layer F.Cu) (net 3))
 (segment (start 147.56 26.755774) (end 150.03 26.79) (width 0.5) (layer F.Cu) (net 3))
 (segment (start 150.03 26.79) (end 150.5 27.21) (width 0.5) (layer F.Cu) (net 3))
 (segment (start 140.84 28.48) (end 144.98 24.95) (width 0.25) (layer F.Cu) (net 2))
 (segment (start 137.36 24.95) (end 136.94 30.455) (width 0.25) (layer F.Cu) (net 17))
 (segment (start 138.94 28.48) (end 138.95 30.76) (width 0.25) (layer F.Cu) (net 1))
 (segment (start 138.95 30.76) (end 138.21 31.64) (width 0.25) (layer F.Cu) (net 1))
 (segment (start 138.21 31.64) (end 136.94 31.725) (width 0.25) (layer F.Cu) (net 1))
 (segment (start 143.01 37.12) (end 143.05 43.66) (width 0.25) (layer F.Cu) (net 10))
 (segment (start 143.01 37.12) (end 142.21 36.31) (width 0.25) (layer F.Cu) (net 10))
 (segment (start 142.21 36.31) (end 142.14 34.265) (width 0.25) (layer F.Cu) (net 10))
 (segment (start 143.05 43.66) (end 144.31 45.19) (width 0.25) (layer F.Cu) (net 10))
 (segment (start 144.31 45.19) (end 145.22 43.79) (width 0.25) (layer F.Cu) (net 10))
 (segment (start 145.22 43.79) (end 146.29 43.3) (width 0.25) (layer F.Cu) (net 10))
 (segment (start 144.37 37.64) (end 145.35 36.02) (width 0.25) (layer F.Cu) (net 11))
 (segment (start 142.14 32.995) (end 143.36 33.55) (width 0.25) (layer F.Cu) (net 11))
 (segment (start 143.36 33.55) (end 143.43 36.25) (width 0.25) (layer F.Cu) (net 11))
 (segment (start 143.43 36.25) (end 144.37 37.64) (width 0.25) (layer F.Cu) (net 11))
 (segment (start 145.35 36.02) (end 146.29 35.73) (width 0.25) (layer F.Cu) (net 11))
 (segment (start 144.35 30.13) (end 145.02 28.45) (width 0.25) (layer F.Cu) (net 14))
 (segment (start 144.35 30.13) (end 142.14 31.725) (width 0.25) (layer F.Cu) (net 14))
 (segment (start 145.02 28.45) (end 146.33 28.18) (width 0.25) (layer F.Cu) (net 14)))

